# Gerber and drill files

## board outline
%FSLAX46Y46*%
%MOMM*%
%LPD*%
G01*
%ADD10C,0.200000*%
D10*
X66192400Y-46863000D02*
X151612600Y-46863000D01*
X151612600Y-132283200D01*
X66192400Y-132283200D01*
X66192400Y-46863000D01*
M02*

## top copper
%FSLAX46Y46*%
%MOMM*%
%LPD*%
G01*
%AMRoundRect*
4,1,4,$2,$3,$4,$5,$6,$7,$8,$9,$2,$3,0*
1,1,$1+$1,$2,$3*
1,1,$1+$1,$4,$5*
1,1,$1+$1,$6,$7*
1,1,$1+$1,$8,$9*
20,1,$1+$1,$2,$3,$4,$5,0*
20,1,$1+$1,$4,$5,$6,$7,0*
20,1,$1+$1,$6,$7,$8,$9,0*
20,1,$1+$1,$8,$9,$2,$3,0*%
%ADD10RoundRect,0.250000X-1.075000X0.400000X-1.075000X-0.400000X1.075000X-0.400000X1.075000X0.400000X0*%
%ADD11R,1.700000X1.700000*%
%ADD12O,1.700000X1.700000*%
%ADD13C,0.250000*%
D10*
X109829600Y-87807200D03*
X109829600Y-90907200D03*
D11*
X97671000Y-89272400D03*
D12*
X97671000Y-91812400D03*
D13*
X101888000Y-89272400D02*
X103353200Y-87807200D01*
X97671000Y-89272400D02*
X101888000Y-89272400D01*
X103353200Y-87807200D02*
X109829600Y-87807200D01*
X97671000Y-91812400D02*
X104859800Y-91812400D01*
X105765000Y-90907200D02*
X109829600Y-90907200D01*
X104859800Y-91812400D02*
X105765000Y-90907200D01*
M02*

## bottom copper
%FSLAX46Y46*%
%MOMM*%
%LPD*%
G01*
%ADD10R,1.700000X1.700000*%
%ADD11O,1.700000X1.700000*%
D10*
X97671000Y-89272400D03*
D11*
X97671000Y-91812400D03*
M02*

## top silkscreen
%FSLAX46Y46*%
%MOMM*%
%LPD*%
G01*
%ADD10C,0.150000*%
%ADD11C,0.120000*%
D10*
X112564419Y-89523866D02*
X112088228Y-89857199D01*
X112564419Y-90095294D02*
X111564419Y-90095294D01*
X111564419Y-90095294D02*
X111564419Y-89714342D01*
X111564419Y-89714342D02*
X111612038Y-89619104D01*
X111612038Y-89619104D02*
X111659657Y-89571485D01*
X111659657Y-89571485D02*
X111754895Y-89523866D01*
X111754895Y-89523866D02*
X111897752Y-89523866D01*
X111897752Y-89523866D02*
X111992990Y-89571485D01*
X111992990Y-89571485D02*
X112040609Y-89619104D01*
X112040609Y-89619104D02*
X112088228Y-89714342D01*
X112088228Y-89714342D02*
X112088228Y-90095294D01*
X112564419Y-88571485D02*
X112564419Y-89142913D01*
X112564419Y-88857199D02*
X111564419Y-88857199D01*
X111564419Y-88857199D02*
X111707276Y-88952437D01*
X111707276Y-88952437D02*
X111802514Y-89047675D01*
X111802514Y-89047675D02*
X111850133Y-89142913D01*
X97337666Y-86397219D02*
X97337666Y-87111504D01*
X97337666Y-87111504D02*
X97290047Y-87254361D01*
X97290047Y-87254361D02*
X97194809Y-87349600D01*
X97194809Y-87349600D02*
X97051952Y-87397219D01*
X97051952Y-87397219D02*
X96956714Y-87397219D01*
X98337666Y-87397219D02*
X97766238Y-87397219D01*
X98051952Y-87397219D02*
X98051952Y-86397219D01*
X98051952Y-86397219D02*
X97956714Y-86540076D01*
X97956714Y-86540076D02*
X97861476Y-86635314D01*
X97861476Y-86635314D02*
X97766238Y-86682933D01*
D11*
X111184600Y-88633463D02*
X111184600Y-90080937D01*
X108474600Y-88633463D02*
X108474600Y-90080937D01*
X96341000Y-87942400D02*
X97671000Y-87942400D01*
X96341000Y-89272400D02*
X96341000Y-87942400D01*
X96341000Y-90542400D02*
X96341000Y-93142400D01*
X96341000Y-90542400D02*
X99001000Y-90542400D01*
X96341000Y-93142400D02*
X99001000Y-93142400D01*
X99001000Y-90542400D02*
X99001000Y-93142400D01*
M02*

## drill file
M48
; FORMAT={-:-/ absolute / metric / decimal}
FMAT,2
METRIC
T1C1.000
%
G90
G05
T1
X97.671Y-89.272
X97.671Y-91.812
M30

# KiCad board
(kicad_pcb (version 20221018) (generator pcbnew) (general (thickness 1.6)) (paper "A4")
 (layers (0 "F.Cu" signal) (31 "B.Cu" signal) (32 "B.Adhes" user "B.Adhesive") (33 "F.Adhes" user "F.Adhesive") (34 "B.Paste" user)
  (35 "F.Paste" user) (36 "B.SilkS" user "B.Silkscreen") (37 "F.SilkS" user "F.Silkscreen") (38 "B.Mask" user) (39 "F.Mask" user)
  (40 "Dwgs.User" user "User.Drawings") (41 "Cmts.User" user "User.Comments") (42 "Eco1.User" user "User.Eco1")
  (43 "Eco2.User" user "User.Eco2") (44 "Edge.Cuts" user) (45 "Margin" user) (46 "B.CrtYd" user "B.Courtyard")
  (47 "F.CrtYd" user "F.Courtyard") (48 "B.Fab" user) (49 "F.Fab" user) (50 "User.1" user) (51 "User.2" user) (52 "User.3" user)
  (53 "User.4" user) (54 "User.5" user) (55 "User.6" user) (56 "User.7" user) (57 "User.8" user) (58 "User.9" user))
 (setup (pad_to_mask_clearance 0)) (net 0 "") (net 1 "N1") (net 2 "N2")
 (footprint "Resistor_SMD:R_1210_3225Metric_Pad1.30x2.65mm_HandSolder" (layer "F.Cu") (at 109.8296 89.3572 -90)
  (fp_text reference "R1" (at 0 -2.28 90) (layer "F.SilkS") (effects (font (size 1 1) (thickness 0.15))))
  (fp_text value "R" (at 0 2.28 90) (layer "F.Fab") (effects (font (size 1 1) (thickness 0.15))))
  (fp_line (start -0.723737 -1.355) (end 0.723737 -1.355) (stroke (width 0.12) (type solid)) (layer "F.SilkS"))
  (fp_line (start -0.723737 1.355) (end 0.723737 1.355) (stroke (width 0.12) (type solid)) (layer "F.SilkS"))
  (pad "1" smd roundrect (at -1.55 0 270) (size 1.3 2.65) (layers "F.Cu" "F.Paste" "F.Mask") (roundrect_rratio 0.192308) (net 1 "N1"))
  (pad "2" smd roundrect (at 1.55 0 270) (size 1.3 2.65) (layers "F.Cu" "F.Paste" "F.Mask") (roundrect_rratio 0.192308) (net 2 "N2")))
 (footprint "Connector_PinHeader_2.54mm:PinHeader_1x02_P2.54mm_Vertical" (layer "F.Cu") (at 97.671 89.2724)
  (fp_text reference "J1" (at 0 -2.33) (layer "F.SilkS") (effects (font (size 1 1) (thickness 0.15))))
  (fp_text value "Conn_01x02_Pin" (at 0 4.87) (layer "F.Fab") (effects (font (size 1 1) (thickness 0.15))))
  (fp_line (start -1.33 -1.33) (end 0 -1.33) (stroke (width 0.12) (type solid)) (layer "F.SilkS"))
  (fp_line (start -1.33 0) (end -1.33 -1.33) (stroke (width 0.12) (type solid)) (layer "F.SilkS"))
  (fp_line (start -1.33 1.27) (end -1.33 3.87) (stroke (width 0.12) (type solid)) (layer "F.SilkS"))
  (fp_line (start -1.33 1.27) (end 1.33 1.27) (stroke (width 0.12) (type solid)) (layer "F.SilkS"))
  (fp_line (start -1.33 3.87) (end 1.33 3.87) (stroke (width 0.12) (type solid)) (layer "F.SilkS"))
  (fp_line (start 1.33 1.27) (end 1.33 3.87) (stroke (width 0.12) (type solid)) (layer "F.SilkS"))
  (pad "1" thru_hole rect (at 0 0) (size 1.7 1.7) (drill 1) (layers "*.Cu" "*.Mask") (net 1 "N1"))
  (pad "2" thru_hole oval (at 0 2.54) (size 1.7 1.7) (drill 1) (layers "*.Cu" "*.Mask") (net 2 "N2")))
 (gr_rect (start 66.1924 46.863) (end 151.6126 132.2832) (stroke (width 0.2) (type default)) (fill none) (layer "Edge.Cuts"))
 (segment (start 101.888 89.2724) (end 103.3532 87.8072) (width 0.25) (layer "F.Cu") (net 1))
 (segment (start 97.671 89.2724) (end 101.888 89.2724) (width 0.25) (layer "F.Cu") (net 1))
 (segment (start 103.3532 87.8072) (end 109.8296 87.8072) (width 0.25) (layer "F.Cu") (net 1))
 (segment (start 97.671 91.8124) (end 104.8598 91.8124) (width 0.25) (layer "F.Cu") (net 2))
 (segment (start 105.765 90.9072) (end 109.8296 90.9072) (width 0.25) (layer "F.Cu") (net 2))
 (segment (start 104.8598 91.8124) (end 105.765 90.9072) (width 0.25) (layer "F.Cu") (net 2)))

